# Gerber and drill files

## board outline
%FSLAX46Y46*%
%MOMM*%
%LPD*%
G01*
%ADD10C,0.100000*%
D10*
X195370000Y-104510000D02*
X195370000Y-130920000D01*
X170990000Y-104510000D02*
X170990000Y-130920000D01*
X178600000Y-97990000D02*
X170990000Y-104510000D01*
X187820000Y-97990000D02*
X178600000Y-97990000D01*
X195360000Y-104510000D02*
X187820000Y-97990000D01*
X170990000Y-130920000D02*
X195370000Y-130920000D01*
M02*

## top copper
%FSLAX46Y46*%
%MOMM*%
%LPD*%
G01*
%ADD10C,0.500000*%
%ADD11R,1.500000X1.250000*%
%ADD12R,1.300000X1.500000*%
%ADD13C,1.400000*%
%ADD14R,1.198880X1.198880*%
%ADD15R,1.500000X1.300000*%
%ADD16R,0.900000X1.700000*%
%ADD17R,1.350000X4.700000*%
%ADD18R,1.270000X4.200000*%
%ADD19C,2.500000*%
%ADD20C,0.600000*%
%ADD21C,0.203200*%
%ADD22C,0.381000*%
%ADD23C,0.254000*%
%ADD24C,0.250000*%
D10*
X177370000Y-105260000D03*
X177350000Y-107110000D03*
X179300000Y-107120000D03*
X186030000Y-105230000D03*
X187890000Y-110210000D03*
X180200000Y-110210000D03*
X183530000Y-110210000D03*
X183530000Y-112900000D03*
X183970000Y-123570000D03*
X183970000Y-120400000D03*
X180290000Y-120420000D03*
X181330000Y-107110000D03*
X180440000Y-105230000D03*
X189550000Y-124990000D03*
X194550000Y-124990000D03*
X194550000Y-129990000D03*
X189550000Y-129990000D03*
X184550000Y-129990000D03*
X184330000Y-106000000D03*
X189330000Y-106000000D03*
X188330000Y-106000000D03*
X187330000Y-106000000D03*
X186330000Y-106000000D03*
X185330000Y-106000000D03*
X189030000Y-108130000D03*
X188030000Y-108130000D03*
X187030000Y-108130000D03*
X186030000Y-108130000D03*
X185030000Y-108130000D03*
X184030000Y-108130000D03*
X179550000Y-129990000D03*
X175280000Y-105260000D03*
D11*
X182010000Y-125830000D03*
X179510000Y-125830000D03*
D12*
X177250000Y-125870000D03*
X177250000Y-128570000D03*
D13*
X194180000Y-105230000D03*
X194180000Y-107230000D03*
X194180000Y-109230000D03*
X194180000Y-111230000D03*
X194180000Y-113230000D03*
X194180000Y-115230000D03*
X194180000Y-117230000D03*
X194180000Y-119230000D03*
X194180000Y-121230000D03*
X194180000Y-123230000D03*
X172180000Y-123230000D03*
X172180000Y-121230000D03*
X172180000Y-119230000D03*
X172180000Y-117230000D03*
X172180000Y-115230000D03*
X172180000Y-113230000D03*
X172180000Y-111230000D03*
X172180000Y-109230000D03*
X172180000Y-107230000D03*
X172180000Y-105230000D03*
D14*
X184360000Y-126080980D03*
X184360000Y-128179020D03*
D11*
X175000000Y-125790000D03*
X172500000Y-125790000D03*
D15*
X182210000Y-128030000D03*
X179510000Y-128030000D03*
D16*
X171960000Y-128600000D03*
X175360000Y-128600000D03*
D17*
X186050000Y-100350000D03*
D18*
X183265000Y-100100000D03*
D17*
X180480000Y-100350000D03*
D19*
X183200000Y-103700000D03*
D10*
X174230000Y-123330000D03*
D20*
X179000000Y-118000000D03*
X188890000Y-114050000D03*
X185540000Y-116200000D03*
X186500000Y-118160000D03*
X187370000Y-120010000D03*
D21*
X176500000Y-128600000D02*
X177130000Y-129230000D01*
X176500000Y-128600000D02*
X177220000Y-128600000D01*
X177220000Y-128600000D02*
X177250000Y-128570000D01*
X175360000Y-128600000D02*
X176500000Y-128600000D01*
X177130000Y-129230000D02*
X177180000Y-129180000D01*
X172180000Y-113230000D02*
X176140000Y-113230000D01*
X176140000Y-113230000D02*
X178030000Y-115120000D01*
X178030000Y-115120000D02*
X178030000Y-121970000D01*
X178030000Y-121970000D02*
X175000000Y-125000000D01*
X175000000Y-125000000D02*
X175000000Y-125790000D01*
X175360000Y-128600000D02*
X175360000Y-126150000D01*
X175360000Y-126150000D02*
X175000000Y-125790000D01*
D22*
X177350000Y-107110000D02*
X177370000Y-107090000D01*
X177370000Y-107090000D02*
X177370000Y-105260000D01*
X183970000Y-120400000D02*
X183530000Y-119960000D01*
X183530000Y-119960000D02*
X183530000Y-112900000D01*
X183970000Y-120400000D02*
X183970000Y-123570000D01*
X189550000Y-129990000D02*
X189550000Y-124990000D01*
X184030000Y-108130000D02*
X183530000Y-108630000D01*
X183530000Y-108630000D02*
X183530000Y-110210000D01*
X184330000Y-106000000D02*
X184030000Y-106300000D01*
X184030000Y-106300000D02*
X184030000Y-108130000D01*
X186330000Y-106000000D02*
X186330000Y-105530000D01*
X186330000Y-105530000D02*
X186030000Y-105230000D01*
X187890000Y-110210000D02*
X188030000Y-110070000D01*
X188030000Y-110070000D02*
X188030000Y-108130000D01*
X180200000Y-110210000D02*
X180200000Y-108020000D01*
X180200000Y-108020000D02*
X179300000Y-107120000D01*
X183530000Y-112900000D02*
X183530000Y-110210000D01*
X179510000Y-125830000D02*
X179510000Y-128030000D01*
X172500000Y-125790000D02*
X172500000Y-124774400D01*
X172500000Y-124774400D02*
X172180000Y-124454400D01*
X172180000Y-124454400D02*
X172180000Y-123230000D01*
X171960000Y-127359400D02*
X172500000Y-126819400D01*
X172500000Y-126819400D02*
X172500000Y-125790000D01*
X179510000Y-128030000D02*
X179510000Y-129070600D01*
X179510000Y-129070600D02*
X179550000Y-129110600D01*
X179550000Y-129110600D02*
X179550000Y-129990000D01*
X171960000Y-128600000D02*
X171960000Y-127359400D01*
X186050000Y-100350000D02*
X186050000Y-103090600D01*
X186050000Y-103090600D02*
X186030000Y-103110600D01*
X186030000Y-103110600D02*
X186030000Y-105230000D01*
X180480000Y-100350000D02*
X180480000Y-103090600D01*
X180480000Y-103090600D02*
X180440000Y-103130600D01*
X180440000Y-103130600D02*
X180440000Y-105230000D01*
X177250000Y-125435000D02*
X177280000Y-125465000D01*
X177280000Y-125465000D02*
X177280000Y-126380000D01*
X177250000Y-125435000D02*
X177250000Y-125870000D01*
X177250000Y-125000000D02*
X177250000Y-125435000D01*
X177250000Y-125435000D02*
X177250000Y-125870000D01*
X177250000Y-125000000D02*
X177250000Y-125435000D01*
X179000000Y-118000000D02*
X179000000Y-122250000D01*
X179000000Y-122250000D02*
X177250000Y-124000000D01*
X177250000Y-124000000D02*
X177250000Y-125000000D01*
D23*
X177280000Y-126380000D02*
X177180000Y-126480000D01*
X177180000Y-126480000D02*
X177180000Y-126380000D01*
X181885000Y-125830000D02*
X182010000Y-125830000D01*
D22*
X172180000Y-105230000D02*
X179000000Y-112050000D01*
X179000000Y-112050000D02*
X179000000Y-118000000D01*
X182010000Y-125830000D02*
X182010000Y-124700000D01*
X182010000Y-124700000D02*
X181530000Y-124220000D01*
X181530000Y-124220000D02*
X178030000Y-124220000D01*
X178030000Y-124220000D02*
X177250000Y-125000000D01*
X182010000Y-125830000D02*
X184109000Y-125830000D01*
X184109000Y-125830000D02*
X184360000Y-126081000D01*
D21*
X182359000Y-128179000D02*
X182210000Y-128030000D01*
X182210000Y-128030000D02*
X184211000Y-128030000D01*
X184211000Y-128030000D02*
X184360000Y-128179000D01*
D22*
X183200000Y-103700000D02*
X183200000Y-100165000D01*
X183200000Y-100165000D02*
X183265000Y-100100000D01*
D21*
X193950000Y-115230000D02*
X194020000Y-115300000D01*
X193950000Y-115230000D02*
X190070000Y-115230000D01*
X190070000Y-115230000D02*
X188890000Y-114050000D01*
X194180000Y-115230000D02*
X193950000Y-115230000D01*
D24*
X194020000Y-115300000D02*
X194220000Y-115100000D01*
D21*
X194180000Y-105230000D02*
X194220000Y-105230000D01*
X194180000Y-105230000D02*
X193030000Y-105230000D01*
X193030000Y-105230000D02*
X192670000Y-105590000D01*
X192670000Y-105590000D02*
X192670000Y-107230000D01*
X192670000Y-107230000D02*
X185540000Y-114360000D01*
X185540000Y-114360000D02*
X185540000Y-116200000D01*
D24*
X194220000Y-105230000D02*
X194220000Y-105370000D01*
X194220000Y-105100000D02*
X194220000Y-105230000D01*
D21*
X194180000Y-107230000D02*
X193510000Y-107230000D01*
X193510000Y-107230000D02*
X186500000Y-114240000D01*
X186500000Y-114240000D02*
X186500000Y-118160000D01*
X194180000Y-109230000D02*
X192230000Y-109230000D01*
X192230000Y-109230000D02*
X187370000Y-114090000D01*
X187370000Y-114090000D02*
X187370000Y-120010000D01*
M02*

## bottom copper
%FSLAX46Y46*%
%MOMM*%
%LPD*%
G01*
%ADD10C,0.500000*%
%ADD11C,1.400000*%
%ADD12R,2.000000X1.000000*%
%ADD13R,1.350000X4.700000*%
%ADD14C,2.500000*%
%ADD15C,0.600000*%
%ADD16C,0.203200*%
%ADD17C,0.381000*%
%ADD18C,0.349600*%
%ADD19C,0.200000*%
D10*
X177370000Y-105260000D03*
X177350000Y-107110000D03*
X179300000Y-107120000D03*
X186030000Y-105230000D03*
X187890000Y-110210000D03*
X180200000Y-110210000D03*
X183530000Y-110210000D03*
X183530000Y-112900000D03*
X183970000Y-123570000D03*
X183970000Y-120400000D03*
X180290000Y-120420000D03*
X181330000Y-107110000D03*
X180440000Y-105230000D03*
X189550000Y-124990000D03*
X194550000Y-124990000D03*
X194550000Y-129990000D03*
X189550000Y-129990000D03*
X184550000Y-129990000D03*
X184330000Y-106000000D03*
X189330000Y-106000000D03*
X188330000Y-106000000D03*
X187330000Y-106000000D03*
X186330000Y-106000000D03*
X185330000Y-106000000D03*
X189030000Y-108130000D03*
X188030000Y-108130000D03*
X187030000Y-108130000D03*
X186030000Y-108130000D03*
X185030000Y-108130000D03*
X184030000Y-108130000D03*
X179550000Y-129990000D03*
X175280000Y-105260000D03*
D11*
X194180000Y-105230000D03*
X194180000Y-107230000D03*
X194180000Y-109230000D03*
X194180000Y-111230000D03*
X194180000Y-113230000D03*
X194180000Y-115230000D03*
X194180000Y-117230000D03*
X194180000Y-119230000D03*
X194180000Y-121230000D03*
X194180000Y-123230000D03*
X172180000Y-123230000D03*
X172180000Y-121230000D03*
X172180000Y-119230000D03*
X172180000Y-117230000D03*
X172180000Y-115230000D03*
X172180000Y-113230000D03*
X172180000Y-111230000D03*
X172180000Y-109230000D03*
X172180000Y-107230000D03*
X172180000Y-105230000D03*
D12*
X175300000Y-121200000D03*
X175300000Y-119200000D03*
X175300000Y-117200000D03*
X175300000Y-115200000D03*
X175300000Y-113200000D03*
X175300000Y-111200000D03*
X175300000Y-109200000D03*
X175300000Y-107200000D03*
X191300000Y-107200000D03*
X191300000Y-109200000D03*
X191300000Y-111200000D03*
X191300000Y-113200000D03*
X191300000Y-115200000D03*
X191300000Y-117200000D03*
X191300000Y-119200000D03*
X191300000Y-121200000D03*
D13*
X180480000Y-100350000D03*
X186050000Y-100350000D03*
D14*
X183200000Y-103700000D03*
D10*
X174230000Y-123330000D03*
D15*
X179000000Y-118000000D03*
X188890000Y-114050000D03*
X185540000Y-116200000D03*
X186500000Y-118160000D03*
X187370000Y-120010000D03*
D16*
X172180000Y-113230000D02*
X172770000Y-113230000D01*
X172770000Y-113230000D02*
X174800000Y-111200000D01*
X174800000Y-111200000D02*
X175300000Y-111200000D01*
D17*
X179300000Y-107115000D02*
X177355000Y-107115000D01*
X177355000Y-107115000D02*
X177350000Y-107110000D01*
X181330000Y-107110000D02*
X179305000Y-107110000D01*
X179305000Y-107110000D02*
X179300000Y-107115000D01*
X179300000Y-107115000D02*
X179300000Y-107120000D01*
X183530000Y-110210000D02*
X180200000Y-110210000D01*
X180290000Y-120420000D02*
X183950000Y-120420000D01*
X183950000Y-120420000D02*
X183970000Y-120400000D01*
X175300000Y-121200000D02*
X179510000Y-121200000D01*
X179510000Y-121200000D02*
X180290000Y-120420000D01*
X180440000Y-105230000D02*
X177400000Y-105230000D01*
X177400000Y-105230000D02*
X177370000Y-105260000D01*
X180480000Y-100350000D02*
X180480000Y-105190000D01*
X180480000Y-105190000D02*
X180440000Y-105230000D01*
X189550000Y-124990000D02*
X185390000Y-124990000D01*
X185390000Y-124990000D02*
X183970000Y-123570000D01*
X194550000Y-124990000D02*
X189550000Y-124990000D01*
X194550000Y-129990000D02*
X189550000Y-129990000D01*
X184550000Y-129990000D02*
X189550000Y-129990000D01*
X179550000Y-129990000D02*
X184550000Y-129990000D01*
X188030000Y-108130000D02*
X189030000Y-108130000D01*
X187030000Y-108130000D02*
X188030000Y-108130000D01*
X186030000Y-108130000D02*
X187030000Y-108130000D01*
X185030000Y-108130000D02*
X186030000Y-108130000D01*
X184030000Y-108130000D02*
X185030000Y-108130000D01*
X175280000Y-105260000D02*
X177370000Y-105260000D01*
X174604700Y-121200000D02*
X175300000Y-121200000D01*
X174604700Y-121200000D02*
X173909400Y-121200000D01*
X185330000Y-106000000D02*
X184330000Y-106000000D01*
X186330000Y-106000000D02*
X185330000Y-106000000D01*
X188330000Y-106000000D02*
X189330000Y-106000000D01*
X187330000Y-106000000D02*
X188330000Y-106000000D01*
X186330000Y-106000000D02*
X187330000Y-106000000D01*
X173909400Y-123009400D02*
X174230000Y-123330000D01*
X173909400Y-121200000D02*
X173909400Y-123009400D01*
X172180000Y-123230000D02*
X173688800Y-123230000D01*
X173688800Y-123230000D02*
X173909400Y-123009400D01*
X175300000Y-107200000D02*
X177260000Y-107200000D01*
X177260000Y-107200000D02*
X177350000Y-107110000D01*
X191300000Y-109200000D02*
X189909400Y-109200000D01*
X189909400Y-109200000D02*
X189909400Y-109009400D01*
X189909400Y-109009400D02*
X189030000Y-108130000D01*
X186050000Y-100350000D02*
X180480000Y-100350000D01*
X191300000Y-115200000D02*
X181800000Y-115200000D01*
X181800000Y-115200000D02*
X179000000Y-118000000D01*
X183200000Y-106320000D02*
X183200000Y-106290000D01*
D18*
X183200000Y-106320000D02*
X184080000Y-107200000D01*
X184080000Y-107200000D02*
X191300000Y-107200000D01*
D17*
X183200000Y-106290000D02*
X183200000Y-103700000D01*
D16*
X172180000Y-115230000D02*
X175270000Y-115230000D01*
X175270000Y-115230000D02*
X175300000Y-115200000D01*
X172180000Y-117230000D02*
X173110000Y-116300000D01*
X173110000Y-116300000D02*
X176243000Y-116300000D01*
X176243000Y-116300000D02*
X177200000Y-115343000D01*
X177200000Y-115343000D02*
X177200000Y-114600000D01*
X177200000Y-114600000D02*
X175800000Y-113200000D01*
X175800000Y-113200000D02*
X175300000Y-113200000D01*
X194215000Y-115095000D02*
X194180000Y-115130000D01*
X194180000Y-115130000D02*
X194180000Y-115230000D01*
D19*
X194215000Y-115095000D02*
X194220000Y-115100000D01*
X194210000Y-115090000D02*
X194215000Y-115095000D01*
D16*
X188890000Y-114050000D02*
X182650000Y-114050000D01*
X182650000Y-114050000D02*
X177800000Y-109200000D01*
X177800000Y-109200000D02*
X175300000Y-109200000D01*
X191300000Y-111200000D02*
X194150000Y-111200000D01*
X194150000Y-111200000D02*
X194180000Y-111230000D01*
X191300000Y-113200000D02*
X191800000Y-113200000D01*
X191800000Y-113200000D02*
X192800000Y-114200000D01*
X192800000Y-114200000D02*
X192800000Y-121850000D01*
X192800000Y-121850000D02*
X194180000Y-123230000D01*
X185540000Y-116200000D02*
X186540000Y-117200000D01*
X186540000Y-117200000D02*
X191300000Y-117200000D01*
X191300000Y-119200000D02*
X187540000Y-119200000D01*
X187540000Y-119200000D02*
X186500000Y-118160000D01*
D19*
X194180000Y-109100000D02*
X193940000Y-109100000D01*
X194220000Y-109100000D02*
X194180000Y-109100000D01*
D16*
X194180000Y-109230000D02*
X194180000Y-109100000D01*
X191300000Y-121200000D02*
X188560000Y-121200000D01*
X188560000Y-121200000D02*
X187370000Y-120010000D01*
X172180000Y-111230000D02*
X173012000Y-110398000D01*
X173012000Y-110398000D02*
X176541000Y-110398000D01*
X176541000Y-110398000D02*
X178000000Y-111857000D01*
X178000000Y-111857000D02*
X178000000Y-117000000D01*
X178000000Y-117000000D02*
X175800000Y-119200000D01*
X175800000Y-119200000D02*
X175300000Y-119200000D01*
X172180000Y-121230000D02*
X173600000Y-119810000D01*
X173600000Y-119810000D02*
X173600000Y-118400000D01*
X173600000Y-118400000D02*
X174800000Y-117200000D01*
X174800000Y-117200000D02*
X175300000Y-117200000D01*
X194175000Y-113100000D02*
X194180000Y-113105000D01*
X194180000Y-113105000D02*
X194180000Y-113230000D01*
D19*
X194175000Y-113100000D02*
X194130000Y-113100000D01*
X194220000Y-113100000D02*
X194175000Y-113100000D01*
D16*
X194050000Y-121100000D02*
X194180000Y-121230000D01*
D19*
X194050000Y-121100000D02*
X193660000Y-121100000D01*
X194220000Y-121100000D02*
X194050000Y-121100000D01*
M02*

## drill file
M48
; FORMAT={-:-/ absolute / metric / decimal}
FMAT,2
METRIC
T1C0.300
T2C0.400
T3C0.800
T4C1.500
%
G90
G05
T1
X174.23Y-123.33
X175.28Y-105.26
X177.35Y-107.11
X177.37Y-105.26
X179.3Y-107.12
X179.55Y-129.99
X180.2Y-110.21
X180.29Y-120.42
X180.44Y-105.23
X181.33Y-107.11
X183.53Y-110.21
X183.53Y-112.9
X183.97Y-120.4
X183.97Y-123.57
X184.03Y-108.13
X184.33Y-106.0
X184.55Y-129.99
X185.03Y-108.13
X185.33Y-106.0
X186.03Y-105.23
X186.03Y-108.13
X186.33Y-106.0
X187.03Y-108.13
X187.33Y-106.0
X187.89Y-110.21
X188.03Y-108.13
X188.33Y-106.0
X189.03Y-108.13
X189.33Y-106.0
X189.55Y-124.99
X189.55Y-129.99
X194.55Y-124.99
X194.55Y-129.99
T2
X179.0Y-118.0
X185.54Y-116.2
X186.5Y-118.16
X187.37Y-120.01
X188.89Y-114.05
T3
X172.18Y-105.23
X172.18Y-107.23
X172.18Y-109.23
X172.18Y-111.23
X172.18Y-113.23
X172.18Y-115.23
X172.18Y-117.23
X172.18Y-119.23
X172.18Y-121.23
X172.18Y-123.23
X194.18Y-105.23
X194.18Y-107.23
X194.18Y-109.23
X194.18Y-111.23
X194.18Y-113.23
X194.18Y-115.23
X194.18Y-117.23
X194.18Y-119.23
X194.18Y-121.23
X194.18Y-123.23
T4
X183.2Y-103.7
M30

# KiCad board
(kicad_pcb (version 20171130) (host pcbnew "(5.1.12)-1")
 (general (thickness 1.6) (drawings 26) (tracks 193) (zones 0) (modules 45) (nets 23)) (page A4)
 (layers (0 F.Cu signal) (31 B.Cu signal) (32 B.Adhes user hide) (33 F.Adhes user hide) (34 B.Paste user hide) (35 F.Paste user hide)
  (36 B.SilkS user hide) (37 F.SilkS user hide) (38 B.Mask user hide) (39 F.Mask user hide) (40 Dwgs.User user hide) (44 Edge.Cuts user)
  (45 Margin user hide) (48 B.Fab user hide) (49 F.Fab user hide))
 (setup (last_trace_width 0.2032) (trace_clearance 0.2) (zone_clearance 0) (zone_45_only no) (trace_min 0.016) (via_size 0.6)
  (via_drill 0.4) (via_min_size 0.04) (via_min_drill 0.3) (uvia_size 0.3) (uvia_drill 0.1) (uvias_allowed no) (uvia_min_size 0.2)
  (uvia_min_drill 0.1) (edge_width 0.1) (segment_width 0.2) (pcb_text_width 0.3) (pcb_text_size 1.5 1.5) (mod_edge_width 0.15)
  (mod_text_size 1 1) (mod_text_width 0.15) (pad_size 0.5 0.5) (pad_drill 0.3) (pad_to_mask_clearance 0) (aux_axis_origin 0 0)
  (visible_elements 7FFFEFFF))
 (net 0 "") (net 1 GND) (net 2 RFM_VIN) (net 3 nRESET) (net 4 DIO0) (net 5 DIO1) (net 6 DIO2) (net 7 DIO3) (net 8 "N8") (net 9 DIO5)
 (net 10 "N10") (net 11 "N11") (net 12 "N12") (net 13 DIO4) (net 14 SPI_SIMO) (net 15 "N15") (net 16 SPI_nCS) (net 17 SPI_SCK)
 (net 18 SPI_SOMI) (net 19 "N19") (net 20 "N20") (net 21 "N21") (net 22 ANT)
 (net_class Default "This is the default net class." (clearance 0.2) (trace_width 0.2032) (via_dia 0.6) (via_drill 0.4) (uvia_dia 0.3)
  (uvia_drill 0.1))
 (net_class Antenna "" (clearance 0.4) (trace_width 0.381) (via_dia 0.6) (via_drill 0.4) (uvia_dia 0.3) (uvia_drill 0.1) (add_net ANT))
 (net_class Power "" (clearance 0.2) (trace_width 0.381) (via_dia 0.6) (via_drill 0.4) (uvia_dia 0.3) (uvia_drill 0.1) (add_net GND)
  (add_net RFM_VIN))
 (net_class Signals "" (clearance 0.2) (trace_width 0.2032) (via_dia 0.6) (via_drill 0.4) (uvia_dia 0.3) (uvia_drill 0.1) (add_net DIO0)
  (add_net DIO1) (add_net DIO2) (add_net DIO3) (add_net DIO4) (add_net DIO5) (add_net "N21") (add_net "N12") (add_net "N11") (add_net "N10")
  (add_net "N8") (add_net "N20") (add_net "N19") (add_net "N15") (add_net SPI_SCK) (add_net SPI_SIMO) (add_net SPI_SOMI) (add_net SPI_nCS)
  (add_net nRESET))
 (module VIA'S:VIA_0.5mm (layer F.Cu) (at 177.37 105.26)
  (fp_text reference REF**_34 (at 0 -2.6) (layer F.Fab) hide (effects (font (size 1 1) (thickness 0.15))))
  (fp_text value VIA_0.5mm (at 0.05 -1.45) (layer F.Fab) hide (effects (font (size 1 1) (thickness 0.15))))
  (pad 1 thru_hole circle (at 0 0) (size 0.5 0.5) (drill 0.3) (layers *.Cu) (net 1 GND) (zone_connect 2)))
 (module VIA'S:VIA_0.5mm (layer F.Cu) (at 177.35 107.11)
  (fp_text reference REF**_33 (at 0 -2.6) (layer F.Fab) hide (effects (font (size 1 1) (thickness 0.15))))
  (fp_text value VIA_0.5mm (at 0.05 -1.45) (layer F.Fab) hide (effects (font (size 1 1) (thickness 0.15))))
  (pad 1 thru_hole circle (at 0 0) (size 0.5 0.5) (drill 0.3) (layers *.Cu) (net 1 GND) (zone_connect 2)))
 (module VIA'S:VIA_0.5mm (layer F.Cu) (at 179.3 107.12)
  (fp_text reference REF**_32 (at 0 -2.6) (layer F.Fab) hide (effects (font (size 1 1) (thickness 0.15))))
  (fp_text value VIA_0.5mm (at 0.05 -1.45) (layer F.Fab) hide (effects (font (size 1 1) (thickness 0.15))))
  (pad 1 thru_hole circle (at 0 0) (size 0.5 0.5) (drill 0.3) (layers *.Cu) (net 1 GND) (zone_connect 2)))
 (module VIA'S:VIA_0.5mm (layer F.Cu) (at 186.03 105.9)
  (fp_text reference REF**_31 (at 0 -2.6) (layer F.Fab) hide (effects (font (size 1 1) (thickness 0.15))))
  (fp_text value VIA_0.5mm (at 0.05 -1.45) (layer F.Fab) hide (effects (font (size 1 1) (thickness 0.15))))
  (pad 1 thru_hole circle (at 0 -0.67) (size 0.5 0.5) (drill 0.3) (layers *.Cu) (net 1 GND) (zone_connect 2)))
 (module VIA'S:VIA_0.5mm (layer F.Cu) (at 187.89 110.29)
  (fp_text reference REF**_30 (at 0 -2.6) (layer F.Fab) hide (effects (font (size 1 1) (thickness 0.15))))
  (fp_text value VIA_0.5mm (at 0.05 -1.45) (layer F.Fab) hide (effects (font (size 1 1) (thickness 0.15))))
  (pad 1 thru_hole circle (at 0 -0.08) (size 0.5 0.5) (drill 0.3) (layers *.Cu) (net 1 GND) (zone_connect 2)))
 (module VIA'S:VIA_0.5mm (layer F.Cu) (at 180.2 110.23)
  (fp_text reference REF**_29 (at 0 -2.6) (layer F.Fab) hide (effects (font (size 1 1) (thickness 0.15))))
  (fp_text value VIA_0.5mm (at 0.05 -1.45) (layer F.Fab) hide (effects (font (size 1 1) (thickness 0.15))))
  (pad 1 thru_hole circle (at 0 -0.02) (size 0.5 0.5) (drill 0.3) (layers *.Cu) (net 1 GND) (zone_connect 2)))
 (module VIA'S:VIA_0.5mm (layer F.Cu) (at 183.53 110.21)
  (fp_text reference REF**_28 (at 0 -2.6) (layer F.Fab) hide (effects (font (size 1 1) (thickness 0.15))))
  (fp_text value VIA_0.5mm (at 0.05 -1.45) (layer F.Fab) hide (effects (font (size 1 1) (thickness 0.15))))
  (pad 1 thru_hole circle (at 0 0) (size 0.5 0.5) (drill 0.3) (layers *.Cu) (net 1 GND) (zone_connect 2)))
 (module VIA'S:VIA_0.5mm (layer F.Cu) (at 183.54 112.9)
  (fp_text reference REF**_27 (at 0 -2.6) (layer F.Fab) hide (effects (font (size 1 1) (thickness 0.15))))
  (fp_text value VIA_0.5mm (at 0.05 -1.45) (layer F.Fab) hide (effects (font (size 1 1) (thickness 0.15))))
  (pad 1 thru_hole circle (at -0.01 0) (size 0.5 0.5) (drill 0.3) (layers *.Cu) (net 1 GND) (zone_connect 2)))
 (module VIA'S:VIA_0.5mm (layer F.Cu) (at 183.97 123.57)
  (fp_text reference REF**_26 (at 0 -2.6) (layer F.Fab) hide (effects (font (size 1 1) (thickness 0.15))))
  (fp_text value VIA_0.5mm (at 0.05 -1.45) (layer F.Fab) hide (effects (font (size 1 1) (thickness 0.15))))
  (pad 1 thru_hole circle (at 0 0) (size 0.5 0.5) (drill 0.3) (layers *.Cu) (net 1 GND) (zone_connect 2)))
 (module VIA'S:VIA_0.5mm (layer F.Cu) (at 183.97 120.4)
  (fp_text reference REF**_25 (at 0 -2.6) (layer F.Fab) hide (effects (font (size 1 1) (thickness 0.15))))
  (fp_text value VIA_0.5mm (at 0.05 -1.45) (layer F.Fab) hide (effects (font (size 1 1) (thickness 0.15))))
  (pad 1 thru_hole circle (at 0 0) (size 0.5 0.5) (drill 0.3) (layers *.Cu) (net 1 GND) (zone_connect 2)))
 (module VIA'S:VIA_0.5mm (layer F.Cu) (at 180.29 120.42)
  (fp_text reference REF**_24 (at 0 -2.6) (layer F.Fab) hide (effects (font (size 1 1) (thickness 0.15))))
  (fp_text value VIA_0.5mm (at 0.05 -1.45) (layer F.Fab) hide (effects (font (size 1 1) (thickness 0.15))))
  (pad 1 thru_hole circle (at 0 0) (size 0.5 0.5) (drill 0.3) (layers *.Cu) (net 1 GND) (zone_connect 2)))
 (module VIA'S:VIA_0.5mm (layer F.Cu) (at 181.33 107.11)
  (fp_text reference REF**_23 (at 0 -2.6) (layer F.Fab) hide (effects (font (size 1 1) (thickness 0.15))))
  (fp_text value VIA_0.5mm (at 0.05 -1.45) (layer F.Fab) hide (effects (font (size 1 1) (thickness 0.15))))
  (pad 1 thru_hole circle (at 0 0) (size 0.5 0.5) (drill 0.3) (layers *.Cu) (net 1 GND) (zone_connect 2)))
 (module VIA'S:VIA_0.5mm (layer F.Cu) (at 180.44 105.23)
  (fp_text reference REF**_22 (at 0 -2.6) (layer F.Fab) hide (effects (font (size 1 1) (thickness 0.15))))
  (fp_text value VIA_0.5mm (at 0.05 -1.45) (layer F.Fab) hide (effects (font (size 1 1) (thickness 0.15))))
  (pad 1 thru_hole circle (at 0 0) (size 0.5 0.5) (drill 0.3) (layers *.Cu) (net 1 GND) (zone_connect 2)))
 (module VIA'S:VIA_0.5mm (layer F.Cu) (at 189.55 124.99)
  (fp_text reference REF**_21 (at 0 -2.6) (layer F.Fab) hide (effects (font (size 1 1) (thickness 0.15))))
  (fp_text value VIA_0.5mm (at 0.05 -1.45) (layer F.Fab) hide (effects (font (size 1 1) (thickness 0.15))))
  (pad 1 thru_hole circle (at 0 0) (size 0.5 0.5) (drill 0.3) (layers *.Cu) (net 1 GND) (zone_connect 2)))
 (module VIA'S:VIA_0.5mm (layer F.Cu) (at 194.55 124.99)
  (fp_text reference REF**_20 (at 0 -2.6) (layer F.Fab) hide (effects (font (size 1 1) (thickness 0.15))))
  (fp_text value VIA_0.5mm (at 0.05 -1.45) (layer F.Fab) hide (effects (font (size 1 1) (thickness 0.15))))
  (pad 1 thru_hole circle (at 0 0) (size 0.5 0.5) (drill 0.3) (layers *.Cu) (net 1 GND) (zone_connect 2)))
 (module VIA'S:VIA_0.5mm (layer F.Cu) (at 194.55 129.99)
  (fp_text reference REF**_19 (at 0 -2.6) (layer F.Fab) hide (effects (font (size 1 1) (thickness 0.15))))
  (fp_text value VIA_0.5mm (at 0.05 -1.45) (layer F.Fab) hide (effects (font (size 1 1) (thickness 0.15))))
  (pad 1 thru_hole circle (at 0 0) (size 0.5 0.5) (drill 0.3) (layers *.Cu) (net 1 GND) (zone_connect 2)))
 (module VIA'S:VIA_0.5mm (layer F.Cu) (at 189.55 129.99)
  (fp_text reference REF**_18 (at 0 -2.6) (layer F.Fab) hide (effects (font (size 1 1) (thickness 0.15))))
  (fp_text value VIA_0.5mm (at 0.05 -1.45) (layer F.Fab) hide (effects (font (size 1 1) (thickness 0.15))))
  (pad 1 thru_hole circle (at 0 0) (size 0.5 0.5) (drill 0.3) (layers *.Cu) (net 1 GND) (zone_connect 2)))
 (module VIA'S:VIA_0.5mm (layer F.Cu) (at 184.55 129.99)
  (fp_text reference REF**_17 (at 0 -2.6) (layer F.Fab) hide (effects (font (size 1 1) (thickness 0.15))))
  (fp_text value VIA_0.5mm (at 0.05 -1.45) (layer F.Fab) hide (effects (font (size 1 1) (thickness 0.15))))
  (pad 1 thru_hole circle (at 0 0) (size 0.5 0.5) (drill 0.3) (layers *.Cu) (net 1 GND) (zone_connect 2)))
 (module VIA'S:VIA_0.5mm (layer F.Cu) (at 184.33 106.67)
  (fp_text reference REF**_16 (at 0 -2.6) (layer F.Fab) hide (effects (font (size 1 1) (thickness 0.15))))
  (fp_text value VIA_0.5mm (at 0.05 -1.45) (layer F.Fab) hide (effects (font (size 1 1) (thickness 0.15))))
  (pad 1 thru_hole circle (at 0 -0.67) (size 0.5 0.5) (drill 0.3) (layers *.Cu) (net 1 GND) (zone_connect 2)))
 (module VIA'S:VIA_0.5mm (layer F.Cu) (at 189.33 106.67)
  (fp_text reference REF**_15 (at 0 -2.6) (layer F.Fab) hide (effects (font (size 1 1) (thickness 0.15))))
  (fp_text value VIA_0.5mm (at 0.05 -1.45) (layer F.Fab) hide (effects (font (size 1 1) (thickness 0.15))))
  (pad 1 thru_hole circle (at 0 -0.67) (size 0.5 0.5) (drill 0.3) (layers *.Cu) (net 1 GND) (zone_connect 2)))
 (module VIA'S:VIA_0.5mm (layer F.Cu) (at 188.33 106.67)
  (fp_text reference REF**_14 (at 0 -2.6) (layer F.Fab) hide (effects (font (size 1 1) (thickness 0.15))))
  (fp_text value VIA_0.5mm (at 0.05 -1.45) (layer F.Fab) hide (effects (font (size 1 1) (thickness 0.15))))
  (pad 1 thru_hole circle (at 0 -0.67) (size 0.5 0.5) (drill 0.3) (layers *.Cu) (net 1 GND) (zone_connect 2)))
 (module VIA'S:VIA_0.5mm (layer F.Cu) (at 187.33 106.67)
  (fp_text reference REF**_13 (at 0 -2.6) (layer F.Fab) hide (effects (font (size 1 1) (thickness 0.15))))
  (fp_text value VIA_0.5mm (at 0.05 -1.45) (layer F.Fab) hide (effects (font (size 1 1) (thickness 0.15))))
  (pad 1 thru_hole circle (at 0 -0.67) (size 0.5 0.5) (drill 0.3) (layers *.Cu) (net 1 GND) (zone_connect 2)))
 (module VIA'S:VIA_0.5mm (layer F.Cu) (at 186.33 106.67)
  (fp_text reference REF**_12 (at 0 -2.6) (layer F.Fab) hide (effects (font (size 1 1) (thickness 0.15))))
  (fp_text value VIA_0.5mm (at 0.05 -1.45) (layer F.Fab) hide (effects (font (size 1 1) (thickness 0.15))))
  (pad 1 thru_hole circle (at 0 -0.67) (size 0.5 0.5) (drill 0.3) (layers *.Cu) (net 1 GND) (zone_connect 2)))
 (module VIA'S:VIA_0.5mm (layer F.Cu) (at 185.33 106.67)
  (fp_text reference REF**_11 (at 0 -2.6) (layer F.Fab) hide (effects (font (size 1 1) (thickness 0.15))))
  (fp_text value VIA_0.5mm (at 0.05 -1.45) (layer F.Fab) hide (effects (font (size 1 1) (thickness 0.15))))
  (pad 1 thru_hole circle (at 0 -0.67) (size 0.5 0.5) (drill 0.3) (layers *.Cu) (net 1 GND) (zone_connect 2)))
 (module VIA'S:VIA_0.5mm (layer F.Cu) (at 189.03 108.13)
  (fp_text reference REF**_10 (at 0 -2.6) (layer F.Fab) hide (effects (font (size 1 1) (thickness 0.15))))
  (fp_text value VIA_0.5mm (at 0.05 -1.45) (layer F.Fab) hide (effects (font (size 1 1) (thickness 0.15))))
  (pad 1 thru_hole circle (at 0 0) (size 0.5 0.5) (drill 0.3) (layers *.Cu) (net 1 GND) (zone_connect 2)))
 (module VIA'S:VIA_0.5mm (layer F.Cu) (at 188.03 108.13)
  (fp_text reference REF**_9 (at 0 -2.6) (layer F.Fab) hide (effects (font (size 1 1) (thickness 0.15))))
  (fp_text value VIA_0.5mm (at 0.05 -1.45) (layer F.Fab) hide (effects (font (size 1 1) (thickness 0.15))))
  (pad 1 thru_hole circle (at 0 0) (size 0.5 0.5) (drill 0.3) (layers *.Cu) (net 1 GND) (zone_connect 2)))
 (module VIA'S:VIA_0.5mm (layer F.Cu) (at 187.03 108.13)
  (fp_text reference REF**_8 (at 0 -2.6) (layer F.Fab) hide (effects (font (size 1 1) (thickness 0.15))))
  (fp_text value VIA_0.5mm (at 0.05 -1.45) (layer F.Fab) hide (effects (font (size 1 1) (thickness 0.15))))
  (pad 1 thru_hole circle (at 0 0) (size 0.5 0.5) (drill 0.3) (layers *.Cu) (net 1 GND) (zone_connect 2)))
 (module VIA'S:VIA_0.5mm (layer F.Cu) (at 186.03 108.13)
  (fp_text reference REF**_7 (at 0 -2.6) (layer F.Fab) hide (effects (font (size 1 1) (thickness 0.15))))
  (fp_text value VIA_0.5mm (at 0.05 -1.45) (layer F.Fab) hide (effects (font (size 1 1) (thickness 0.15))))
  (pad 1 thru_hole circle (at 0 0) (size 0.5 0.5) (drill 0.3) (layers *.Cu) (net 1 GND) (zone_connect 2)))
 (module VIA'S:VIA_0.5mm (layer F.Cu) (at 185.03 108.13)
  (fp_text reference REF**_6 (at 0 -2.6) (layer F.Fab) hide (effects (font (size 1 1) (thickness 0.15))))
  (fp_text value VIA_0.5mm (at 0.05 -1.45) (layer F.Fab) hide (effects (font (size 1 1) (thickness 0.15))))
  (pad 1 thru_hole circle (at 0 0) (size 0.5 0.5) (drill 0.3) (layers *.Cu) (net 1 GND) (zone_connect 2)))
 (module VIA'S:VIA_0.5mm (layer F.Cu) (at 184.03 108.13)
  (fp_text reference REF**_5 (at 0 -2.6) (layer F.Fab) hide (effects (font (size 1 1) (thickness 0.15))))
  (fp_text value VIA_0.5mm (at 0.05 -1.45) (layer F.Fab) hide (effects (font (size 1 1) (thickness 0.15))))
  (pad 1 thru_hole circle (at 0 0) (size 0.5 0.5) (drill 0.3) (layers *.Cu) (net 1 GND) (zone_connect 2)))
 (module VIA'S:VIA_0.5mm (layer F.Cu) (at 179.55 129.99)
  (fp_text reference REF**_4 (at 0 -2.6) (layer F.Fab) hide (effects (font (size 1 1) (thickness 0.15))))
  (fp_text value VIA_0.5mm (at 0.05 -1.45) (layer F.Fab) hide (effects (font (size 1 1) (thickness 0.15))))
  (pad 1 thru_hole circle (at 0 0) (size 0.5 0.5) (drill 0.3) (layers *.Cu) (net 1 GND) (zone_connect 2)))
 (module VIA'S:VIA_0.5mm (layer F.Cu) (at 175.28 105.26)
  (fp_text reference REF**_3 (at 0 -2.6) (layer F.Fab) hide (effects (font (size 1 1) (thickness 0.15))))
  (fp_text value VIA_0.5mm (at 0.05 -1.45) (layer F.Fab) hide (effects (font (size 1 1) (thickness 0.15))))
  (pad 1 thru_hole circle (at 0 0) (size 0.5 0.5) (drill 0.3) (layers *.Cu) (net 1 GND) (zone_connect 2)))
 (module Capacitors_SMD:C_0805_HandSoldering (layer F.Cu) (at 180.76 125.83 180)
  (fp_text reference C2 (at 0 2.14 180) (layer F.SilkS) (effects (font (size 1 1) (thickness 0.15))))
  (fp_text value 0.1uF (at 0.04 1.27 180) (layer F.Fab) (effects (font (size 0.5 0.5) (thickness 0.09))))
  (pad 1 smd rect (at -1.25 0 180) (size 1.5 1.25) (layers F.Cu F.Paste F.Mask) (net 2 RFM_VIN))
  (pad 2 smd rect (at 1.25 0 180) (size 1.5 1.25) (layers F.Cu F.Paste F.Mask) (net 1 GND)))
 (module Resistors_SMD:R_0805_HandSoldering (layer F.Cu) (at 177.25 127.22 270)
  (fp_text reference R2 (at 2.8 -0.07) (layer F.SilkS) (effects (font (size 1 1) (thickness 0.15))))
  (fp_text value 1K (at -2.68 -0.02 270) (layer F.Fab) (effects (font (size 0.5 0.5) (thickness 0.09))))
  (pad 1 smd rect (at -1.35 0 270) (size 1.5 1.3) (layers F.Cu F.Paste F.Mask) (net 2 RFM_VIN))
  (pad 2 smd rect (at 1.35 0 270) (size 1.5 1.3) (layers F.Cu F.Paste F.Mask) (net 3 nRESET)))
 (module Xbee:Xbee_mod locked (layer F.Cu) (at 172.18 105.23)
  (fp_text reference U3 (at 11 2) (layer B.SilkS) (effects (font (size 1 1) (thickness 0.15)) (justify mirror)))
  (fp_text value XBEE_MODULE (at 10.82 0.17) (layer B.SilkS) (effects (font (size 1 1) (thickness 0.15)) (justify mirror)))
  (pad 20 thru_hole circle (at 22 0) (size 1.4 1.4) (drill 0.8) (layers *.Cu *.Mask) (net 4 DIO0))
  (pad 19 thru_hole circle (at 22 2) (size 1.4 1.4) (drill 0.8) (layers *.Cu *.Mask) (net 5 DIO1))
  (pad 18 thru_hole circle (at 22 4) (size 1.4 1.4) (drill 0.8) (layers *.Cu *.Mask) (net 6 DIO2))
  (pad 17 thru_hole circle (at 22 6) (size 1.4 1.4) (drill 0.8) (layers *.Cu *.Mask) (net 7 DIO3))
  (pad 16 thru_hole circle (at 22 8) (size 1.4 1.4) (drill 0.8) (layers *.Cu *.Mask) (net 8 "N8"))
  (pad 15 thru_hole circle (at 22 10) (size 1.4 1.4) (drill 0.8) (layers *.Cu *.Mask) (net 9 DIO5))
  (pad 14 thru_hole circle (at 22 12) (size 1.4 1.4) (drill 0.8) (layers *.Cu *.Mask) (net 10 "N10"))
  (pad 13 thru_hole circle (at 22 14) (size 1.4 1.4) (drill 0.8) (layers *.Cu *.Mask) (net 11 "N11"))
  (pad 12 thru_hole circle (at 22 16) (size 1.4 1.4) (drill 0.8) (layers *.Cu *.Mask) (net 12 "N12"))
  (pad 11 thru_hole circle (at 22 18) (size 1.4 1.4) (drill 0.8) (layers *.Cu *.Mask) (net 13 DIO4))
  (pad 10 thru_hole circle (at 0 18) (size 1.4 1.4) (drill 0.8) (layers *.Cu *.Mask) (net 1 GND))
  (pad 9 thru_hole circle (at 0 16) (size 1.4 1.4) (drill 0.8) (layers *.Cu *.Mask) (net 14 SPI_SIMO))
  (pad 8 thru_hole circle (at 0 14) (size 1.4 1.4) (drill 0.8) (layers *.Cu *.Mask) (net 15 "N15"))
  (pad 7 thru_hole circle (at 0 12) (size 1.4 1.4) (drill 0.8) (layers *.Cu *.Mask) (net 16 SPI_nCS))
  (pad 6 thru_hole circle (at 0 10) (size 1.4 1.4) (drill 0.8) (layers *.Cu *.Mask) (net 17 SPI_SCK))
  (pad 5 thru_hole circle (at 0 8) (size 1.4 1.4) (drill 0.8) (layers *.Cu *.Mask) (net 3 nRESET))
  (pad 4 thru_hole circle (at 0 6) (size 1.4 1.4) (drill 0.8) (layers *.Cu *.Mask) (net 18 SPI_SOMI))
  (pad 3 thru_hole circle (at 0 4) (size 1.4 1.4) (drill 0.8) (layers *.Cu *.Mask) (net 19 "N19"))
  (pad 2 thru_hole circle (at 0 2) (size 1.4 1.4) (drill 0.8) (layers *.Cu *.Mask) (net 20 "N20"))
  (pad 1 thru_hole circle (at 0 0) (size 1.4 1.4) (drill 0.8) (layers *.Cu *.Mask) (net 2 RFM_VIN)))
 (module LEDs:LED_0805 (layer F.Cu) (at 184.36 127.13 90)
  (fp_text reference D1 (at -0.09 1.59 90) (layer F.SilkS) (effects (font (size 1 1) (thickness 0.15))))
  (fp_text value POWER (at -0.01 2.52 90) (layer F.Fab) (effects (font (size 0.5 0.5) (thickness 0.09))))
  (pad 2 smd rect (at 1.04902 0 270) (size 1.19888 1.19888) (layers F.Cu F.Paste F.Mask) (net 2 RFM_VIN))
  (pad 1 smd rect (at -1.04902 0 270) (size 1.19888 1.19888) (layers F.Cu F.Paste F.Mask) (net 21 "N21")))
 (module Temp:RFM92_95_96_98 (layer B.Cu) (at 175.3 121.2)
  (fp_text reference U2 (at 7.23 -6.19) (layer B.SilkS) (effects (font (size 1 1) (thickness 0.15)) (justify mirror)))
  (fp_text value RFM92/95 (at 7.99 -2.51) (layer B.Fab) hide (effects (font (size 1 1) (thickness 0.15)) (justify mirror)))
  (pad 1 smd rect (at 0 0) (size 2 1) (layers B.Cu B.Paste B.Mask) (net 1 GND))
  (pad 2 smd rect (at 0 -2) (size 2 1) (layers B.Cu B.Paste B.Mask) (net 18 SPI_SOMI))
  (pad 3 smd rect (at 0 -4) (size 2 1) (layers B.Cu B.Paste B.Mask) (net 14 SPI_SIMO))
  (pad 4 smd rect (at 0 -6) (size 2 1) (layers B.Cu B.Paste B.Mask) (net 17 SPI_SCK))
  (pad 5 smd rect (at 0 -8) (size 2 1) (layers B.Cu B.Paste B.Mask) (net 16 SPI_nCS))
  (pad 6 smd rect (at 0 -10) (size 2 1) (layers B.Cu B.Paste B.Mask) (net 3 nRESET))
  (pad 7 smd rect (at 0 -12) (size 2 1) (layers B.Cu B.Paste B.Mask) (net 9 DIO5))
  (pad 8 smd rect (at 0 -14) (size 2 1) (layers B.Cu B.Paste B.Mask) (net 1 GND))
  (pad 9 smd rect (at 16 -14) (size 2 1) (layers B.Cu B.Paste B.Mask) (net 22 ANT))
  (pad 10 smd rect (at 16 -12) (size 2 1) (layers B.Cu B.Paste B.Mask) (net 1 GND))
  (pad 11 smd rect (at 16 -10) (size 2 1) (layers B.Cu B.Paste B.Mask) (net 7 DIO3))
  (pad 12 smd rect (at 16 -8) (size 2 1) (layers B.Cu B.Paste B.Mask) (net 13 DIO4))
  (pad 13 smd rect (at 16 -6) (size 2 1) (layers B.Cu B.Paste B.Mask) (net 2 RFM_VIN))
  (pad 14 smd rect (at 16 -4) (size 2 1) (layers B.Cu B.Paste B.Mask) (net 4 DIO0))
  (pad 15 smd rect (at 16 -2) (size 2 1) (layers B.Cu B.Paste B.Mask) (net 5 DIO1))
  (pad 16 smd rect (at 16 0) (size 2 1) (layers B.Cu B.Paste B.Mask) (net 6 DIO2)))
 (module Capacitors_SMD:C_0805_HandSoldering (layer F.Cu) (at 173.75 125.79 180)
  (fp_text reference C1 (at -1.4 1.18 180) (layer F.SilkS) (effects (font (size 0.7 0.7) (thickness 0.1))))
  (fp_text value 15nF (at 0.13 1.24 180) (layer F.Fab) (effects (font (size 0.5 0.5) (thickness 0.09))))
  (pad 1 smd rect (at -1.25 0 180) (size 1.5 1.25) (layers F.Cu F.Paste F.Mask) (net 3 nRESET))
  (pad 2 smd rect (at 1.25 0 180) (size 1.5 1.25) (layers F.Cu F.Paste F.Mask) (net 1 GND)))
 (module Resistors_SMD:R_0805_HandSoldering (layer F.Cu) (at 180.86 128.03 180)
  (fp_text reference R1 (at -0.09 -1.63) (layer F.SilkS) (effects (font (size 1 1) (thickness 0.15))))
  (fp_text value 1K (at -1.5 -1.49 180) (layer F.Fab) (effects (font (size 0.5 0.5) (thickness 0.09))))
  (pad 1 smd rect (at -1.35 0 180) (size 1.5 1.3) (layers F.Cu F.Paste F.Mask) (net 21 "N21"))
  (pad 2 smd rect (at 1.35 0 180) (size 1.5 1.3) (layers F.Cu F.Paste F.Mask) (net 1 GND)))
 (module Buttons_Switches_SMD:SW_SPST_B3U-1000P (layer F.Cu) (at 173.66 128.6)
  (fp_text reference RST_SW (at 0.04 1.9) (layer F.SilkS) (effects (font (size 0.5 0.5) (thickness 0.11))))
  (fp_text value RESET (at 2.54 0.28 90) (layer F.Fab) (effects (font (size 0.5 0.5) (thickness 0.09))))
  (pad 1 smd rect (at -1.7 0) (size 0.9 1.7) (layers F.Cu F.Paste F.Mask) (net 1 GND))
  (pad 2 smd rect (at 1.7 0) (size 0.9 1.7) (layers F.Cu F.Paste F.Mask) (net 3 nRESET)))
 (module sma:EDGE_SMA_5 (layer F.Cu) (at 186.05 100.35 270)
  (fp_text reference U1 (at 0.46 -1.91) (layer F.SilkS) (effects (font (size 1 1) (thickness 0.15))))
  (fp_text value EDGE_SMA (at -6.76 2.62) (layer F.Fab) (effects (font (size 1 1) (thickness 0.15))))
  (pad 5 smd rect (at 0 5.57 270) (size 4.7 1.35) (layers B.Cu F.Paste F.Mask) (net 1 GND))
  (pad 3 smd rect (at 0 0 270) (size 4.7 1.35) (layers B.Cu F.Paste F.Mask) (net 1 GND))
  (pad 2 smd rect (at 0 0 270) (size 4.7 1.35) (layers F.Cu F.Paste F.Mask) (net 1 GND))
  (pad 1 smd rect (at -0.25 2.785 270) (size 4.2 1.27) (layers F.Cu F.Paste F.Mask) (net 22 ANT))
  (pad 4 smd rect (at 0 5.57 270) (size 4.7 1.35) (layers F.Cu F.Paste F.Mask) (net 1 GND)))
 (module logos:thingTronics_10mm (layer F.Cu) (at 182.23 117.37)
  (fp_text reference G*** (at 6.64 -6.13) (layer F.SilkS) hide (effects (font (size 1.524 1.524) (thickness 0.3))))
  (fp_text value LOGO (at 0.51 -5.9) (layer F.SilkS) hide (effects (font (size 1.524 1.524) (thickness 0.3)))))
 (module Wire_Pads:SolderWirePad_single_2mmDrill (layer F.Cu) (at 183.2 103.7)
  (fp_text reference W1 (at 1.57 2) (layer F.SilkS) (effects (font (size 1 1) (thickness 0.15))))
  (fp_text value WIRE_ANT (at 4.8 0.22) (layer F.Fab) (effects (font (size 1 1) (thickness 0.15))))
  (pad 1 thru_hole circle (at 0 0) (size 2.5 2.5) (drill 1.5) (layers *.Cu F.Mask) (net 22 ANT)))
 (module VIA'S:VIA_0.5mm (layer F.Cu) (at 174.23 123.33)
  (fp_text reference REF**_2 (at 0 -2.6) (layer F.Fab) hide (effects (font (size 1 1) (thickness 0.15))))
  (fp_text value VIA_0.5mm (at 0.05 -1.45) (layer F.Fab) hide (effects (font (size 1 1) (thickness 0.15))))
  (pad 1 thru_hole circle (at 0 0) (size 0.5 0.5) (drill 0.3) (layers *.Cu) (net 1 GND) (zone_connect 2)))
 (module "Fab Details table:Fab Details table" (layer F.Cu) (at 127.11 93.44)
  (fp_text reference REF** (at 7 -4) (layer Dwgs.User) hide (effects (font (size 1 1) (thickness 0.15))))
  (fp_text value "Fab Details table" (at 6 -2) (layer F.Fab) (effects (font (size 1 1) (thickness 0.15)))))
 (gr_line (start 195.37 104.51) (end 195.37 130.92) (layer Edge.Cuts) (width 0.1))
 (gr_line (start 170.99 104.51) (end 170.99 130.92) (layer Edge.Cuts) (width 0.1))
 (gr_line (start 178.6 97.99) (end 170.99 104.51) (layer Edge.Cuts) (width 0.1))
 (gr_line (start 187.82 97.99) (end 178.6 97.99) (layer Edge.Cuts) (width 0.1))
 (gr_line (start 195.36 104.51) (end 187.82 97.99) (layer Edge.Cuts) (width 0.1))
 (gr_line (start 170.99 130.92) (end 195.37 130.92) (layer Edge.Cuts) (width 0.1))
 (segment (start 176.5 128.6) (end 177.13 129.23) (width 0.2032) (layer F.Cu) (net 3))
 (segment (start 176.5 128.6) (end 177.22 128.6) (width 0.2032) (layer F.Cu) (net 3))
 (segment (start 177.22 128.6) (end 177.25 128.57) (width 0.2032) (layer F.Cu) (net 3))
 (segment (start 175.36 128.6) (end 176.5 128.6) (width 0.2032) (layer F.Cu) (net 3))
 (segment (start 172.18 113.23) (end 172.77 113.23) (width 0.2032) (layer B.Cu) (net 3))
 (segment (start 172.77 113.23) (end 174.8 111.2) (width 0.2032) (layer B.Cu) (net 3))
 (segment (start 174.8 111.2) (end 175.3 111.2) (width 0.2032) (layer B.Cu) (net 3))
 (segment (start 177.13 129.23) (end 177.18 129.18) (width 0.2032) (layer F.Cu) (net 3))
 (segment (start 172.18 113.23) (end 176.14 113.23) (width 0.2032) (layer F.Cu) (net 3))
 (segment (start 176.14 113.23) (end 178.03 115.12) (width 0.2032) (layer F.Cu) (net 3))
 (segment (start 178.03 115.12) (end 178.03 121.97) (width 0.2032) (layer F.Cu) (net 3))
 (segment (start 178.03 121.97) (end 175 125) (width 0.2032) (layer F.Cu) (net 3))
 (segment (start 175 125) (end 175 125.79) (width 0.2032) (layer F.Cu) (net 3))
 (segment (start 175.36 128.6) (end 175.36 126.15) (width 0.2032) (layer F.Cu) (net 3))
 (segment (start 175.36 126.15) (end 175 125.79) (width 0.2032) (layer F.Cu) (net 3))
 (segment (start 177.35 107.11) (end 177.37 107.09) (width 0.381) (layer F.Cu) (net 1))
 (segment (start 177.37 107.09) (end 177.37 105.26) (width 0.381) (layer F.Cu) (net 1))
 (segment (start 179.3 107.115) (end 177.355 107.115) (width 0.381) (layer B.Cu) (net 1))
 (segment (start 177.355 107.115) (end 177.35 107.11) (width 0.381) (layer B.Cu) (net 1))
 (segment (start 181.33 107.11) (end 179.305 107.11) (width 0.381) (layer B.Cu) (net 1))
 (segment (start 179.305 107.11) (end 179.3 107.115) (width 0.381) (layer B.Cu) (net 1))
 (segment (start 179.3 107.115) (end 179.3 107.12) (width 0.381) (layer B.Cu) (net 1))
 (segment (start 183.53 110.21) (end 180.2 110.21) (width 0.381) (layer B.Cu) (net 1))
 (segment (start 183.97 120.4) (end 183.53 119.96) (width 0.381) (layer F.Cu) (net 1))
 (segment (start 183.53 119.96) (end 183.53 112.9) (width 0.381) (layer F.Cu) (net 1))
 (segment (start 183.97 120.4) (end 183.97 123.57) (width 0.381) (layer F.Cu) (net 1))
 (segment (start 180.29 120.42) (end 183.95 120.42) (width 0.381) (layer B.Cu) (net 1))
 (segment (start 183.95 120.42) (end 183.97 120.4) (width 0.381) (layer B.Cu) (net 1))
 (segment (start 175.3 121.2) (end 179.51 121.2) (width 0.381) (layer B.Cu) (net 1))
 (segment (start 179.51 121.2) (end 180.29 120.42) (width 0.381) (layer B.Cu) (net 1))
 (segment (start 180.44 105.23) (end 177.4 105.23) (width 0.381) (layer B.Cu) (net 1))
 (segment (start 177.4 105.23) (end 177.37 105.26) (width 0.381) (layer B.Cu) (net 1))
 (segment (start 180.48 100.35) (end 180.48 105.19) (width 0.381) (layer B.Cu) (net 1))
 (segment (start 180.48 105.19) (end 180.44 105.23) (width 0.381) (layer B.Cu) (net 1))
 (segment (start 189.55 124.99) (end 185.39 124.99) (width 0.381) (layer B.Cu) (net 1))
 (segment (start 185.39 124.99) (end 183.97 123.57) (width 0.381) (layer B.Cu) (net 1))
 (segment (start 194.55 124.99) (end 189.55 124.99) (width 0.381) (layer B.Cu) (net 1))
 (segment (start 194.55 129.99) (end 189.55 129.99) (width 0.381) (layer B.Cu) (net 1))
 (segment (start 189.55 129.99) (end 189.55 124.99) (width 0.381) (layer F.Cu) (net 1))
 (segment (start 184.55 129.99) (end 189.55 129.99) (width 0.381) (layer B.Cu) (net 1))
 (segment (start 179.55 129.99) (end 184.55 129.99) (width 0.381) (layer B.Cu) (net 1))
 (segment (start 184.03 108.13) (end 183.53 108.63) (width 0.381) (layer F.Cu) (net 1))
 (segment (start 183.53 108.63) (end 183.53 110.21) (width 0.381) (layer F.Cu) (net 1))
 (segment (start 184.33 106) (end 184.03 106.3) (width 0.381) (layer F.Cu) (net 1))
 (segment (start 184.03 106.3) (end 184.03 108.13) (width 0.381) (layer F.Cu) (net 1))
 (segment (start 188.03 108.13) (end 189.03 108.13) (width 0.381) (layer B.Cu) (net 1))
 (segment (start 187.03 108.13) (end 188.03 108.13) (width 0.381) (layer B.Cu) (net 1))
 (segment (start 186.03 108.13) (end 187.03 108.13) (width 0.381) (layer B.Cu) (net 1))
 (segment (start 185.03 108.13) (end 186.03 108.13) (width 0.381) (layer B.Cu) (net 1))
 (segment (start 184.03 108.13) (end 185.03 108.13) (width 0.381) (layer B.Cu) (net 1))
 (segment (start 175.28 105.26) (end 177.37 105.26) (width 0.381) (layer B.Cu) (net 1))
 (segment (start 174.6047 121.2) (end 175.3 121.2) (width 0.381) (layer B.Cu) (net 1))
 (segment (start 174.6047 121.2) (end 173.9094 121.2) (width 0.381) (layer B.Cu) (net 1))
 (segment (start 186.33 106) (end 186.33 105.53) (width 0.381) (layer F.Cu) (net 1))
 (segment (start 186.33 105.53) (end 186.03 105.23) (width 0.381) (layer F.Cu) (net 1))
 (segment (start 185.33 106) (end 184.33 106) (width 0.381) (layer B.Cu) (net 1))
 (segment (start 186.33 106) (end 185.33 106) (width 0.381) (layer B.Cu) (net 1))
 (segment (start 188.33 106) (end 189.33 106) (width 0.381) (layer B.Cu) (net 1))
 (segment (start 187.33 106) (end 188.33 106) (width 0.381) (layer B.Cu) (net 1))
 (segment (start 186.33 106) (end 187.33 106) (width 0.381) (layer B.Cu) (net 1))
 (segment (start 187.89 110.21) (end 188.03 110.07) (width 0.381) (layer F.Cu) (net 1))
 (segment (start 188.03 110.07) (end 188.03 108.13) (width 0.381) (layer F.Cu) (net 1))
 (segment (start 180.2 110.21) (end 180.2 108.02) (width 0.381) (layer F.Cu) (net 1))
 (segment (start 180.2 108.02) (end 179.3 107.12) (width 0.381) (layer F.Cu) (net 1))
 (segment (start 183.53 112.9) (end 183.53 110.21) (width 0.381) (layer F.Cu) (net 1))
 (segment (start 179.51 125.83) (end 179.51 128.03) (width 0.381) (layer F.Cu) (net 1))
 (segment (start 172.5 125.79) (end 172.5 124.7744) (width 0.381) (layer F.Cu) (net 1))
 (segment (start 172.5 124.7744) (end 172.18 124.4544) (width 0.381) (layer F.Cu) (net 1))
 (segment (start 172.18 124.4544) (end 172.18 123.23) (width 0.381) (layer F.Cu) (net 1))
 (segment (start 171.96 127.3594) (end 172.5 126.8194) (width 0.381) (layer F.Cu) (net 1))
 (segment (start 172.5 126.8194) (end 172.5 125.79) (width 0.381) (layer F.Cu) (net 1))
 (segment (start 179.51 128.03) (end 179.51 129.0706) (width 0.381) (layer F.Cu) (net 1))
 (segment (start 179.51 129.0706) (end 179.55 129.1106) (width 0.381) (layer F.Cu) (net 1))
 (segment (start 179.55 129.1106) (end 179.55 129.99) (width 0.381) (layer F.Cu) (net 1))
 (segment (start 173.9094 123.0094) (end 174.23 123.33) (width 0.381) (layer B.Cu) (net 1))
 (segment (start 173.9094 121.2) (end 173.9094 123.0094) (width 0.381) (layer B.Cu) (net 1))
 (segment (start 172.18 123.23) (end 173.6888 123.23) (width 0.381) (layer B.Cu) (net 1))
 (segment (start 173.6888 123.23) (end 173.9094 123.0094) (width 0.381) (layer B.Cu) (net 1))
 (segment (start 175.3 107.2) (end 177.26 107.2) (width 0.381) (layer B.Cu) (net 1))
 (segment (start 177.26 107.2) (end 177.35 107.11) (width 0.381) (layer B.Cu) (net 1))
 (segment (start 191.3 109.2) (end 189.9094 109.2) (width 0.381) (layer B.Cu) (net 1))
 (segment (start 189.9094 109.2) (end 189.9094 109.0094) (width 0.381) (layer B.Cu) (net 1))
 (segment (start 189.9094 109.0094) (end 189.03 108.13) (width 0.381) (layer B.Cu) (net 1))
 (segment (start 171.96 128.6) (end 171.96 127.3594) (width 0.381) (layer F.Cu) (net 1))
 (segment (start 186.05 100.35) (end 180.48 100.35) (width 0.381) (layer B.Cu) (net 1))
 (segment (start 186.05 100.35) (end 186.05 103.0906) (width 0.381) (layer F.Cu) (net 1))
 (segment (start 186.05 103.0906) (end 186.03 103.1106) (width 0.381) (layer F.Cu) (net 1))
 (segment (start 186.03 103.1106) (end 186.03 105.23) (width 0.381) (layer F.Cu) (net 1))
 (segment (start 180.48 100.35) (end 180.48 103.0906) (width 0.381) (layer F.Cu) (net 1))
 (segment (start 180.48 103.0906) (end 180.44 103.1306) (width 0.381) (layer F.Cu) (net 1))
 (segment (start 180.44 103.1306) (end 180.44 105.23) (width 0.381) (layer F.Cu) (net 1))
 (segment (start 177.25 125.435) (end 177.28 125.465) (width 0.381) (layer F.Cu) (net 2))
 (segment (start 177.28 125.465) (end 177.28 126.38) (width 0.381) (layer F.Cu) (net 2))
 (segment (start 177.25 125.435) (end 177.25 125.87) (width 0.381) (layer F.Cu) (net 2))
 (segment (start 177.25 125) (end 177.25 125.435) (width 0.381) (layer F.Cu) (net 2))
 (segment (start 177.25 125.435) (end 177.25 125.87) (width 0.381) (layer F.Cu) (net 2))
 (segment (start 177.25 125) (end 177.25 125.435) (width 0.381) (layer F.Cu) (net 2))
 (segment (start 179 118) (end 179 122.25) (width 0.381) (layer F.Cu) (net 2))
 (segment (start 179 122.25) (end 177.25 124) (width 0.381) (layer F.Cu) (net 2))
 (segment (start 177.25 124) (end 177.25 125) (width 0.381) (layer F.Cu) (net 2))
 (segment (start 177.28 126.38) (end 177.18 126.48) (width 0.254) (layer F.Cu) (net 2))
 (segment (start 177.18 126.48) (end 177.18 126.38) (width 0.254) (layer F.Cu) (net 2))
 (segment (start 181.885 125.83) (end 182.01 125.83) (width 0.254) (layer F.Cu) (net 2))
 (segment (start 172.18 105.23) (end 179 112.05) (width 0.381) (layer F.Cu) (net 2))
 (segment (start 179 112.05) (end 179 118) (width 0.381) (layer F.Cu) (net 2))
 (segment (start 182.01 125.83) (end 182.01 124.7) (width 0.381) (layer F.Cu) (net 2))
 (segment (start 182.01 124.7) (end 181.53 124.22) (width 0.381) (layer F.Cu) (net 2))
 (segment (start 181.53 124.22) (end 178.03 124.22) (width 0.381) (layer F.Cu) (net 2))
 (segment (start 178.03 124.22) (end 177.25 125) (width 0.381) (layer F.Cu) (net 2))
 (segment (start 191.3 115.2) (end 181.8 115.2) (width 0.381) (layer B.Cu) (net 2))
 (segment (start 181.8 115.2) (end 179 118) (width 0.381) (layer B.Cu) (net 2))
 (segment (start 182.01 125.83) (end 184.109 125.83) (width 0.381) (layer F.Cu) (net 2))
 (segment (start 184.109 125.83) (end 184.36 126.081) (width 0.381) (layer F.Cu) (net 2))
 (via (at 179 118) (size 0.6) (layers F.Cu B.Cu) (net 2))
 (segment (start 182.359 128.179) (end 182.21 128.03) (width 0.2032) (layer F.Cu) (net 21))
 (segment (start 182.21 128.03) (end 184.211 128.03) (width 0.2032) (layer F.Cu) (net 21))
 (segment (start 184.211 128.03) (end 184.36 128.179) (width 0.2032) (layer F.Cu) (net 21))
 (segment (start 183.2 106.32) (end 183.2 106.29) (width 0.381) (layer B.Cu) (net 22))
 (segment (start 183.2 106.32) (end 184.08 107.2) (width 0.3496) (layer B.Cu) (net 22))
 (segment (start 184.08 107.2) (end 191.3 107.2) (width 0.3496) (layer B.Cu) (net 22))
 (segment (start 183.2 106.29) (end 183.2 103.7) (width 0.381) (layer B.Cu) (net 22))
 (segment (start 183.2 103.7) (end 183.2 100.165) (width 0.381) (layer F.Cu) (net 22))
 (segment (start 183.2 100.165) (end 183.265 100.1) (width 0.381) (layer F.Cu) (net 22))
 (segment (start 172.18 115.23) (end 175.27 115.23) (width 0.2032) (layer B.Cu) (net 17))
 (segment (start 175.27 115.23) (end 175.3 115.2) (width 0.2032) (layer B.Cu) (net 17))
 (segment (start 172.18 117.23) (end 173.11 116.3) (width 0.2032) (layer B.Cu) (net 16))
 (segment (start 173.11 116.3) (end 176.243 116.3) (width 0.2032) (layer B.Cu) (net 16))
 (segment (start 176.243 116.3) (end 177.2 115.343) (width 0.2032) (layer B.Cu) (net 16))
 (segment (start 177.2 115.343) (end 177.2 114.6) (width 0.2032) (layer B.Cu) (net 16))
 (segment (start 177.2 114.6) (end 175.8 113.2) (width 0.2032) (layer B.Cu) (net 16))
 (segment (start 175.8 113.2) (end 175.3 113.2) (width 0.2032) (layer B.Cu) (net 16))
 (segment (start 194.215 115.095) (end 194.18 115.13) (width 0.2032) (layer B.Cu) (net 9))
 (segment (start 194.18 115.13) (end 194.18 115.23) (width 0.2032) (layer B.Cu) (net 9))
 (segment (start 194.215 115.095) (end 194.22 115.1) (width 0.2) (layer B.Cu) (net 9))
 (segment (start 194.21 115.09) (end 194.215 115.095) (width 0.2) (layer B.Cu) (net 9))
 (segment (start 193.95 115.23) (end 194.02 115.3) (width 0.2032) (layer F.Cu) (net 9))
 (segment (start 193.95 115.23) (end 190.07 115.23) (width 0.2032) (layer F.Cu) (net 9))
 (segment (start 190.07 115.23) (end 188.89 114.05) (width 0.2032) (layer F.Cu) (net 9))
 (segment (start 194.18 115.23) (end 193.95 115.23) (width 0.2032) (layer F.Cu) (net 9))
 (segment (start 194.02 115.3) (end 194.22 115.1) (width 0.25) (layer F.Cu) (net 9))
 (segment (start 188.89 114.05) (end 182.65 114.05) (width 0.2032) (layer B.Cu) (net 9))
 (segment (start 182.65 114.05) (end 177.8 109.2) (width 0.2032) (layer B.Cu) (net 9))
 (segment (start 177.8 109.2) (end 175.3 109.2) (width 0.2032) (layer B.Cu) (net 9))
 (via (at 188.89 114.05) (size 0.6) (layers F.Cu B.Cu) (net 9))
 (segment (start 191.3 111.2) (end 194.15 111.2) (width 0.2032) (layer B.Cu) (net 7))
 (segment (start 194.15 111.2) (end 194.18 111.23) (width 0.2032) (layer B.Cu) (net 7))
 (segment (start 191.3 113.2) (end 191.8 113.2) (width 0.2032) (layer B.Cu) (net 13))
 (segment (start 191.8 113.2) (end 192.8 114.2) (width 0.2032) (layer B.Cu) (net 13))
 (segment (start 192.8 114.2) (end 192.8 121.85) (width 0.2032) (layer B.Cu) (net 13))
 (segment (start 192.8 121.85) (end 194.18 123.23) (width 0.2032) (layer B.Cu) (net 13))
 (segment (start 194.18 105.23) (end 194.22 105.23) (width 0.2032) (layer F.Cu) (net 4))
 (segment (start 194.18 105.23) (end 193.03 105.23) (width 0.2032) (layer F.Cu) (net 4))
 (segment (start 193.03 105.23) (end 192.67 105.59) (width 0.2032) (layer F.Cu) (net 4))
 (segment (start 192.67 105.59) (end 192.67 107.23) (width 0.2032) (layer F.Cu) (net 4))
 (segment (start 192.67 107.23) (end 185.54 114.36) (width 0.2032) (layer F.Cu) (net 4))
 (segment (start 185.54 114.36) (end 185.54 116.2) (width 0.2032) (layer F.Cu) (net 4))
 (segment (start 194.22 105.23) (end 194.22 105.37) (width 0.25) (layer F.Cu) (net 4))
 (segment (start 194.22 105.1) (end 194.22 105.23) (width 0.25) (layer F.Cu) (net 4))
 (segment (start 185.54 116.2) (end 186.54 117.2) (width 0.2032) (layer B.Cu) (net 4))
 (segment (start 186.54 117.2) (end 191.3 117.2) (width 0.2032) (layer B.Cu) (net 4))
 (via (at 185.54 116.2) (size 0.6) (layers F.Cu B.Cu) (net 4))
 (segment (start 191.3 119.2) (end 187.54 119.2) (width 0.2032) (layer B.Cu) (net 5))
 (segment (start 187.54 119.2) (end 186.5 118.16) (width 0.2032) (layer B.Cu) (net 5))
 (segment (start 194.18 107.23) (end 193.51 107.23) (width 0.2032) (layer F.Cu) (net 5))
 (segment (start 193.51 107.23) (end 186.5 114.24) (width 0.2032) (layer F.Cu) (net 5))
 (segment (start 186.5 114.24) (end 186.5 118.16) (width 0.2032) (layer F.Cu) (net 5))
 (via (at 186.5 118.16) (size 0.6) (layers F.Cu B.Cu) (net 5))
 (segment (start 194.18 109.1) (end 193.94 109.1) (width 0.2) (layer B.Cu) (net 6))
 (segment (start 194.22 109.1) (end 194.18 109.1) (width 0.2) (layer B.Cu) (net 6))
 (segment (start 194.18 109.23) (end 194.18 109.1) (width 0.2032) (layer B.Cu) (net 6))
 (segment (start 191.3 121.2) (end 188.56 121.2) (width 0.2032) (layer B.Cu) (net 6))
 (segment (start 188.56 121.2) (end 187.37 120.01) (width 0.2032) (layer B.Cu) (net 6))
 (segment (start 194.18 109.23) (end 192.23 109.23) (width 0.2032) (layer F.Cu) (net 6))
 (segment (start 192.23 109.23) (end 187.37 114.09) (width 0.2032) (layer F.Cu) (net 6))
 (segment (start 187.37 114.09) (end 187.37 120.01) (width 0.2032) (layer F.Cu) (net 6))
 (via (at 187.37 120.01) (size 0.6) (layers F.Cu B.Cu) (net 6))
 (segment (start 172.18 111.23) (end 173.012 110.398) (width 0.2032) (layer B.Cu) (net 18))
 (segment (start 173.012 110.398) (end 176.541 110.398) (width 0.2032) (layer B.Cu) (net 18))
 (segment (start 176.541 110.398) (end 178 111.857) (width 0.2032) (layer B.Cu) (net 18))
 (segment (start 178 111.857) (end 178 117) (width 0.2032) (layer B.Cu) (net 18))
 (segment (start 178 117) (end 175.8 119.2) (width 0.2032) (layer B.Cu) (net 18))
 (segment (start 175.8 119.2) (end 175.3 119.2) (width 0.2032) (layer B.Cu) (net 18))
 (segment (start 172.18 121.23) (end 173.6 119.81) (width 0.2032) (layer B.Cu) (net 14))
 (segment (start 173.6 119.81) (end 173.6 118.4) (width 0.2032) (layer B.Cu) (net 14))
 (segment (start 173.6 118.4) (end 174.8 117.2) (width 0.2032) (layer B.Cu) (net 14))
 (segment (start 174.8 117.2) (end 175.3 117.2) (width 0.2032) (layer B.Cu) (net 14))
 (segment (start 194.175 113.1) (end 194.18 113.105) (width 0.2032) (layer B.Cu) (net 8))
 (segment (start 194.18 113.105) (end 194.18 113.23) (width 0.2032) (layer B.Cu) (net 8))
 (segment (start 194.175 113.1) (end 194.13 113.1) (width 0.2) (layer B.Cu) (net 8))
 (segment (start 194.22 113.1) (end 194.175 113.1) (width 0.2) (layer B.Cu) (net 8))
 (segment (start 194.05 121.1) (end 194.18 121.23) (width 0.2032) (layer B.Cu) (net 12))
 (segment (start 194.05 121.1) (end 193.66 121.1) (width 0.2) (layer B.Cu) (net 12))
 (segment (start 194.22 121.1) (end 194.05 121.1) (width 0.2) (layer B.Cu) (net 12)))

